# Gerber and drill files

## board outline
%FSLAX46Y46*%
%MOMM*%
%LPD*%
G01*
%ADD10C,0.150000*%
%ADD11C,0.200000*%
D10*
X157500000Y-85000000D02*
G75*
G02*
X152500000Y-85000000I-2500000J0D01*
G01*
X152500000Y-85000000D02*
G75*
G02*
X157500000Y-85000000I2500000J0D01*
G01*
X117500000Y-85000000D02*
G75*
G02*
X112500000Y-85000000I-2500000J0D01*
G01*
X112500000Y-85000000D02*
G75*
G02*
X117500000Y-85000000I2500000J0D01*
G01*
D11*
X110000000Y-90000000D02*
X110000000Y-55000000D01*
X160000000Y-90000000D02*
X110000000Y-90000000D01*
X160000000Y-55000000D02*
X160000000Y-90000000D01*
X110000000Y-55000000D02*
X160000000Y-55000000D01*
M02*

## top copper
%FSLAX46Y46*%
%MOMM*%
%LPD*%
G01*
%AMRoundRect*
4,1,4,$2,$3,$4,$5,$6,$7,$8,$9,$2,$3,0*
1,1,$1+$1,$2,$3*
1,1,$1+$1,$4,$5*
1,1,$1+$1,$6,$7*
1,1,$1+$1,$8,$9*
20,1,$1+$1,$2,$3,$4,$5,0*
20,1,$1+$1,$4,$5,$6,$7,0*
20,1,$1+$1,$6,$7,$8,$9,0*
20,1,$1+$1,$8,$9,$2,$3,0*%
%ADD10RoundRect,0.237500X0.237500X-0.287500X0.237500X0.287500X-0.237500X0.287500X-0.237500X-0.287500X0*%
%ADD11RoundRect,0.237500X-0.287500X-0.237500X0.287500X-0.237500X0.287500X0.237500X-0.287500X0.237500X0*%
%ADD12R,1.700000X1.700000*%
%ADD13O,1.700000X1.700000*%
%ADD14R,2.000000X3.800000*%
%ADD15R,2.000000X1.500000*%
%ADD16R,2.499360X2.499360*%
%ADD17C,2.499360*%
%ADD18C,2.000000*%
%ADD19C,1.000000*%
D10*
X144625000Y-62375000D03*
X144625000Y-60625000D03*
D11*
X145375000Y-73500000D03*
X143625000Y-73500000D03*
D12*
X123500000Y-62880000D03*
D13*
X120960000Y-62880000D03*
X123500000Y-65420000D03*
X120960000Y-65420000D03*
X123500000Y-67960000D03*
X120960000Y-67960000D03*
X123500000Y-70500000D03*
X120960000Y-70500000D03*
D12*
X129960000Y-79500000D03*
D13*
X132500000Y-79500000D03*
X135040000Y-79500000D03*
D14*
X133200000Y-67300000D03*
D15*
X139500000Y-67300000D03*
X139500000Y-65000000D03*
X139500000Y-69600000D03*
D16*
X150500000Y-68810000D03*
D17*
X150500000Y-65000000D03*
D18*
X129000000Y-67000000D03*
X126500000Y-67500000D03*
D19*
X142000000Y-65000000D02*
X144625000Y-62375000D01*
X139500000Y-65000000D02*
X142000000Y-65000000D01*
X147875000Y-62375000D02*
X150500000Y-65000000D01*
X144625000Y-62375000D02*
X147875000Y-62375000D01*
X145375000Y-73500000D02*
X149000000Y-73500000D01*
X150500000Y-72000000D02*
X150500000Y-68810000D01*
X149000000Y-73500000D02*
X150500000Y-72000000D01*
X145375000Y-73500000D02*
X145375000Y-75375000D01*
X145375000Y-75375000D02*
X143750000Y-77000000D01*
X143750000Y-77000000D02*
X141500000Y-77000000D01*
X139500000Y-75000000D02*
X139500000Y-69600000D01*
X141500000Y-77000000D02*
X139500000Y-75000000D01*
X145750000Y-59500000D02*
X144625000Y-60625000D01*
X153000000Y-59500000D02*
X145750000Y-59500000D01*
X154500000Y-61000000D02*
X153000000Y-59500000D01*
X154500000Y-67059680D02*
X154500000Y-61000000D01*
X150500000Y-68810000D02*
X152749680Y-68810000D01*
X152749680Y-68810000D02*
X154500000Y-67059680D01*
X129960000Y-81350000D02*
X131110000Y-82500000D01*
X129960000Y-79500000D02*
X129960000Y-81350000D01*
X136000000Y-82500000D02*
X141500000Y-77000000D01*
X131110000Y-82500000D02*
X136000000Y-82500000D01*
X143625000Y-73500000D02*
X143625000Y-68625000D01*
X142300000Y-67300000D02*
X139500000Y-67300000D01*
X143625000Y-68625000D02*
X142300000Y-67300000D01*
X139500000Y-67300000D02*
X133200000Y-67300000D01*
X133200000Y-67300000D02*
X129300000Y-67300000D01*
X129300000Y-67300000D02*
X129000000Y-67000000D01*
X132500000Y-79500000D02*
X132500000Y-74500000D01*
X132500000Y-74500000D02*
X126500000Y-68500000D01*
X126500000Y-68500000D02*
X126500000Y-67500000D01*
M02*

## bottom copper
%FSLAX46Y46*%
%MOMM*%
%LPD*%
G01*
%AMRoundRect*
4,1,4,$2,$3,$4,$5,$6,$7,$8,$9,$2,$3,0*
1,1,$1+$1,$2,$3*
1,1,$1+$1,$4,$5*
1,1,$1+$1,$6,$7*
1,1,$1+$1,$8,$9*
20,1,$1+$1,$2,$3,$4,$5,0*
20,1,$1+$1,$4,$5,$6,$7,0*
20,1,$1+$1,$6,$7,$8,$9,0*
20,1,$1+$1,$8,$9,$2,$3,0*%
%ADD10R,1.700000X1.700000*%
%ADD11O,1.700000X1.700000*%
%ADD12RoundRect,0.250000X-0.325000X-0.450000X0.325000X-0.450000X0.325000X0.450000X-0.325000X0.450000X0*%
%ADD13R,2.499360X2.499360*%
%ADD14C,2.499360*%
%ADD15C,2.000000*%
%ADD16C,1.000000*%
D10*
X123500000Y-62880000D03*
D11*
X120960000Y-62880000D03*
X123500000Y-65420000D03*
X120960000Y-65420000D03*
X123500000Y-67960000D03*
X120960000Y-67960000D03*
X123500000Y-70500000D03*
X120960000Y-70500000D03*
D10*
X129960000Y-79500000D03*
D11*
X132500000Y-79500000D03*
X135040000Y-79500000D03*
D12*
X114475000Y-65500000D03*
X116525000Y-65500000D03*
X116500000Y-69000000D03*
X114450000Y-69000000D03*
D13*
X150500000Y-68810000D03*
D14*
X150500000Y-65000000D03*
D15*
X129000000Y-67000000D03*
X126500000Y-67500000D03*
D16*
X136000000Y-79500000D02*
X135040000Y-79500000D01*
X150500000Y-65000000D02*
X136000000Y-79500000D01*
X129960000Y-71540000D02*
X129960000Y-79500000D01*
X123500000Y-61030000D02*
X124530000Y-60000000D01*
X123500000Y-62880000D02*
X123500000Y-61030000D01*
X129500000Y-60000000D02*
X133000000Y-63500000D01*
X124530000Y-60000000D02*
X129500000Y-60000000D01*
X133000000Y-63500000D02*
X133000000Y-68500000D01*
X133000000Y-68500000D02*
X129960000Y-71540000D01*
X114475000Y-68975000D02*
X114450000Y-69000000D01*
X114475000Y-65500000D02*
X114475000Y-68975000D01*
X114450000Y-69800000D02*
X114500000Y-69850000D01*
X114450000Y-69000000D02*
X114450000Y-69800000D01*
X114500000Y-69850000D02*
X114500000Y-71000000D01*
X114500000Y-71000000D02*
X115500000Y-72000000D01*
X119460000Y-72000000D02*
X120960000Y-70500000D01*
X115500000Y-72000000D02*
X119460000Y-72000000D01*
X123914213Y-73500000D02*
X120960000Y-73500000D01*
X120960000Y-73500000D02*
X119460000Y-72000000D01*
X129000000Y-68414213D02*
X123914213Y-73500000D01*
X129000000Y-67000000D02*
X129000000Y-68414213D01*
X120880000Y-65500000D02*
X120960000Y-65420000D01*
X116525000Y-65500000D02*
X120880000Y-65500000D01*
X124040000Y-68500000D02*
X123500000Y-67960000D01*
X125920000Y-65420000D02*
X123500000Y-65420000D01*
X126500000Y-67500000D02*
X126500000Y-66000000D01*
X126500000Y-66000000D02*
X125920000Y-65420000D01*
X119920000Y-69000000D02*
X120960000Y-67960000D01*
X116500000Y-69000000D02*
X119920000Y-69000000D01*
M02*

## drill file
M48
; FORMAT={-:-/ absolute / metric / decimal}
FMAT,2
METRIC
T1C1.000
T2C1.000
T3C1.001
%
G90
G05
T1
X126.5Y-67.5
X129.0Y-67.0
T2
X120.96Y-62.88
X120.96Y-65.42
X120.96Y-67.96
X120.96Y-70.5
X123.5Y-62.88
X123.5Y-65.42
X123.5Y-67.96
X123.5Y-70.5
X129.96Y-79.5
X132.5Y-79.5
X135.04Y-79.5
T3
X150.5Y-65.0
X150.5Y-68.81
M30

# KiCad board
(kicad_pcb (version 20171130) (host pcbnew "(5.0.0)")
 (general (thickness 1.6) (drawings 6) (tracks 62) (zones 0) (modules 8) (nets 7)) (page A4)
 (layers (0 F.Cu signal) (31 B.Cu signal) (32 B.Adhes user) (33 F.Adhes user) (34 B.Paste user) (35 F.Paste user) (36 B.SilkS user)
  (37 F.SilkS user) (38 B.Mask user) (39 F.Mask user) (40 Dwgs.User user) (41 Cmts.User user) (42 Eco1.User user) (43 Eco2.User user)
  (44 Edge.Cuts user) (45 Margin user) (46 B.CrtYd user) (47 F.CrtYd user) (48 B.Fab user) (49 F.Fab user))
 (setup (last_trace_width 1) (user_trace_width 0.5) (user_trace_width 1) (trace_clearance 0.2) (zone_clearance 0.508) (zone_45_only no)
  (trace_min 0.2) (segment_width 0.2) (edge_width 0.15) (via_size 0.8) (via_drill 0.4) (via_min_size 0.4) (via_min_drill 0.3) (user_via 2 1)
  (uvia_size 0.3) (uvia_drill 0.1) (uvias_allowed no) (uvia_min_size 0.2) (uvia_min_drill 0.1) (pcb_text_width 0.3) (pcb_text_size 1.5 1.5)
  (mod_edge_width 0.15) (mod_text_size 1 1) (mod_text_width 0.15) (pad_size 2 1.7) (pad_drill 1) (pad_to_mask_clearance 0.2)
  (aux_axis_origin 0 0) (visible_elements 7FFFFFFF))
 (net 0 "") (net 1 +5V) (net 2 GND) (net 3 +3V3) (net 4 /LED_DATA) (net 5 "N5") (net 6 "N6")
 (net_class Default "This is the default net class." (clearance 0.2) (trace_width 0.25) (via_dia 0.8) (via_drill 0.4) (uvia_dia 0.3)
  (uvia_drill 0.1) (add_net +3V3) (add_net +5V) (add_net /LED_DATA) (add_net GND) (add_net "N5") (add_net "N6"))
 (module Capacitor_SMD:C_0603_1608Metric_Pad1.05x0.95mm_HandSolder (layer F.Cu) (at 144.625 61.5 90)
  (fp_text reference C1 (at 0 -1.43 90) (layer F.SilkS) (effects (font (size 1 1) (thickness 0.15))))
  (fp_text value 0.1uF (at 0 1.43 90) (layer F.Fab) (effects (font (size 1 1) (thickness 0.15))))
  (pad 1 smd roundrect (at -0.875 0 90) (size 1.05 0.95) (layers F.Cu F.Paste F.Mask) (roundrect_rratio 0.25) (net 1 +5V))
  (pad 2 smd roundrect (at 0.875 0 90) (size 1.05 0.95) (layers F.Cu F.Paste F.Mask) (roundrect_rratio 0.25) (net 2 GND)))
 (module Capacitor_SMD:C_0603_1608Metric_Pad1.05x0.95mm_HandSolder (layer F.Cu) (at 144.5 73.5)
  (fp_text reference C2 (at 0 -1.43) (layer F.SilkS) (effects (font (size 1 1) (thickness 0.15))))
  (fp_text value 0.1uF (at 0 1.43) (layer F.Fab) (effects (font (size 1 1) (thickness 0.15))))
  (pad 2 smd roundrect (at 0.875 0) (size 1.05 0.95) (layers F.Cu F.Paste F.Mask) (roundrect_rratio 0.25) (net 2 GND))
  (pad 1 smd roundrect (at -0.875 0) (size 1.05 0.95) (layers F.Cu F.Paste F.Mask) (roundrect_rratio 0.25) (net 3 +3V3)))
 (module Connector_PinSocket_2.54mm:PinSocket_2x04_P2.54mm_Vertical (layer F.Cu) (at 123.5 62.88)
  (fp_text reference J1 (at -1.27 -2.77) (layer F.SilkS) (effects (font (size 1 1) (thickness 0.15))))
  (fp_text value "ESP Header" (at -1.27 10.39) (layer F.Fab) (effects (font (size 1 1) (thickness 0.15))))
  (pad 1 thru_hole rect (at 0 0) (size 1.7 1.7) (drill 1) (layers *.Cu *.Mask) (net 2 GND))
  (pad 2 thru_hole oval (at -2.54 0) (size 1.7 1.7) (drill 1) (layers *.Cu *.Mask))
  (pad 3 thru_hole oval (at 0 2.54) (size 1.7 1.7) (drill 1) (layers *.Cu *.Mask) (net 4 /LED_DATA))
  (pad 4 thru_hole oval (at -2.54 2.54) (size 1.7 1.7) (drill 1) (layers *.Cu *.Mask) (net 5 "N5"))
  (pad 5 thru_hole oval (at 0 5.08) (size 1.7 1.7) (drill 1) (layers *.Cu *.Mask))
  (pad 6 thru_hole oval (at -2.54 5.08) (size 1.7 1.7) (drill 1) (layers *.Cu *.Mask) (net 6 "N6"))
  (pad 7 thru_hole oval (at 0 7.62) (size 1.7 1.7) (drill 1) (layers *.Cu *.Mask))
  (pad 8 thru_hole oval (at -2.54 7.62) (size 1.7 1.7) (drill 1) (layers *.Cu *.Mask) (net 3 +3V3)))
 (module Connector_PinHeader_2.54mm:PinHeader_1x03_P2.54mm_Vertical (layer F.Cu) (at 129.96 79.5 90)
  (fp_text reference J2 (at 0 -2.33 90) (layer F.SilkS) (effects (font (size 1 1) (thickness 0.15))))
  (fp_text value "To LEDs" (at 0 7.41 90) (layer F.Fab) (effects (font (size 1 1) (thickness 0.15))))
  (pad 1 thru_hole rect (at 0 0 90) (size 1.7 1.7) (drill 1) (layers *.Cu *.Mask) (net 2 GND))
  (pad 2 thru_hole oval (at 0 2.54 90) (size 1.7 1.7) (drill 1) (layers *.Cu *.Mask) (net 4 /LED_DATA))
  (pad 3 thru_hole oval (at 0 5.08 90) (size 1.7 1.7) (drill 1) (layers *.Cu *.Mask) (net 1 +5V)))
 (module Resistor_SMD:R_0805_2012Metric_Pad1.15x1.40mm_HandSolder (layer B.Cu) (at 115.5 65.5)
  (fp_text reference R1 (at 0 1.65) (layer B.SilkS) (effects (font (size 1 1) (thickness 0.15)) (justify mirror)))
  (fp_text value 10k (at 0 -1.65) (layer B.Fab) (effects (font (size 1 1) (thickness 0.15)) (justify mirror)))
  (pad 1 smd roundrect (at -1.025 0) (size 1.15 1.4) (layers B.Cu B.Paste B.Mask) (roundrect_rratio 0.217391) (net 3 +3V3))
  (pad 2 smd roundrect (at 1.025 0) (size 1.15 1.4) (layers B.Cu B.Paste B.Mask) (roundrect_rratio 0.217391) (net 5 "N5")))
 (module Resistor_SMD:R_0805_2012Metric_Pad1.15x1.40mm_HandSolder (layer B.Cu) (at 115.475 69)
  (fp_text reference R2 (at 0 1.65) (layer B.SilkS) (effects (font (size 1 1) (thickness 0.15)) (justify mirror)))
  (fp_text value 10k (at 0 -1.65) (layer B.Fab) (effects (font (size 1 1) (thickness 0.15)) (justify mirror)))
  (pad 2 smd roundrect (at 1.025 0) (size 1.15 1.4) (layers B.Cu B.Paste B.Mask) (roundrect_rratio 0.217391) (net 6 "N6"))
  (pad 1 smd roundrect (at -1.025 0) (size 1.15 1.4) (layers B.Cu B.Paste B.Mask) (roundrect_rratio 0.217391) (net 3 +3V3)))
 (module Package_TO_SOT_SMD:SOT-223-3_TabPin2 (layer F.Cu) (at 136.35 67.3 180)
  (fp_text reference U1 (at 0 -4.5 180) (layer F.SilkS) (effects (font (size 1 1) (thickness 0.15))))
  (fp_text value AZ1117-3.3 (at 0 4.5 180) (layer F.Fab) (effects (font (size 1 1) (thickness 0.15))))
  (pad 2 smd rect (at 3.15 0 180) (size 2 3.8) (layers F.Cu F.Paste F.Mask) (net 3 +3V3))
  (pad 2 smd rect (at -3.15 0 180) (size 2 1.5) (layers F.Cu F.Paste F.Mask) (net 3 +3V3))
  (pad 3 smd rect (at -3.15 2.3 180) (size 2 1.5) (layers F.Cu F.Paste F.Mask) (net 1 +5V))
  (pad 1 smd rect (at -3.15 -2.3 180) (size 2 1.5) (layers F.Cu F.Paste F.Mask) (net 2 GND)))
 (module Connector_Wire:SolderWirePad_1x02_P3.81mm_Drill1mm (layer F.Cu) (at 150.5 68.81 90)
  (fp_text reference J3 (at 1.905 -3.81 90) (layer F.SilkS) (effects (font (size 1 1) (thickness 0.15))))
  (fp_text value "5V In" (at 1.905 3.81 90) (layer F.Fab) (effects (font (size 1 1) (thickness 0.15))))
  (pad 1 thru_hole rect (at 0 0 90) (size 2.49936 2.49936) (drill 1.00076) (layers *.Cu *.Mask) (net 2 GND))
  (pad 2 thru_hole circle (at 3.81 0 90) (size 2.49936 2.49936) (drill 1.00076) (layers *.Cu *.Mask) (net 1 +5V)))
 (gr_circle (center 155 85) (end 157.5 85) (layer Edge.Cuts) (width 0.15))
 (gr_circle (center 115 85) (end 117.5 85) (layer Edge.Cuts) (width 0.15))
 (gr_line (start 110 90) (end 110 55) (layer Edge.Cuts) (width 0.2))
 (gr_line (start 160 90) (end 110 90) (layer Edge.Cuts) (width 0.2))
 (gr_line (start 160 55) (end 160 90) (layer Edge.Cuts) (width 0.2))
 (gr_line (start 110 55) (end 160 55) (layer Edge.Cuts) (width 0.2))
 (segment (start 142 65) (end 144.625 62.375) (width 1) (layer F.Cu) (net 1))
 (segment (start 139.5 65) (end 142 65) (width 1) (layer F.Cu) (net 1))
 (segment (start 147.875 62.375) (end 150.5 65) (width 1) (layer F.Cu) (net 1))
 (segment (start 144.625 62.375) (end 147.875 62.375) (width 1) (layer F.Cu) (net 1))
 (segment (start 136 79.5) (end 135.04 79.5) (width 1) (layer B.Cu) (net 1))
 (segment (start 150.5 65) (end 136 79.5) (width 1) (layer B.Cu) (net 1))
 (segment (start 145.375 73.5) (end 149 73.5) (width 1) (layer F.Cu) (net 2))
 (segment (start 150.5 72) (end 150.5 68.81) (width 1) (layer F.Cu) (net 2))
 (segment (start 149 73.5) (end 150.5 72) (width 1) (layer F.Cu) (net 2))
 (segment (start 145.375 73.5) (end 145.375 75.375) (width 1) (layer F.Cu) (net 2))
 (segment (start 145.375 75.375) (end 143.75 77) (width 1) (layer F.Cu) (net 2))
 (segment (start 143.75 77) (end 141.5 77) (width 1) (layer F.Cu) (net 2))
 (segment (start 139.5 75) (end 139.5 69.6) (width 1) (layer F.Cu) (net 2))
 (segment (start 141.5 77) (end 139.5 75) (width 1) (layer F.Cu) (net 2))
 (segment (start 145.75 59.5) (end 144.625 60.625) (width 1) (layer F.Cu) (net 2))
 (segment (start 153 59.5) (end 145.75 59.5) (width 1) (layer F.Cu) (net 2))
 (segment (start 154.5 61) (end 153 59.5) (width 1) (layer F.Cu) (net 2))
 (segment (start 154.5 67.05968) (end 154.5 61) (width 1) (layer F.Cu) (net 2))
 (segment (start 150.5 68.81) (end 152.74968 68.81) (width 1) (layer F.Cu) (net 2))
 (segment (start 152.74968 68.81) (end 154.5 67.05968) (width 1) (layer F.Cu) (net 2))
 (segment (start 129.96 81.35) (end 131.11 82.5) (width 1) (layer F.Cu) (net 2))
 (segment (start 129.96 79.5) (end 129.96 81.35) (width 1) (layer F.Cu) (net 2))
 (segment (start 136 82.5) (end 141.5 77) (width 1) (layer F.Cu) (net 2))
 (segment (start 131.11 82.5) (end 136 82.5) (width 1) (layer F.Cu) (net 2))
 (segment (start 129.96 71.54) (end 129.96 79.5) (width 1) (layer B.Cu) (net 2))
 (segment (start 123.5 61.03) (end 124.53 60) (width 1) (layer B.Cu) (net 2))
 (segment (start 123.5 62.88) (end 123.5 61.03) (width 1) (layer B.Cu) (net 2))
 (segment (start 129.5 60) (end 133 63.5) (width 1) (layer B.Cu) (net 2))
 (segment (start 124.53 60) (end 129.5 60) (width 1) (layer B.Cu) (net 2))
 (segment (start 133 63.5) (end 133 68.5) (width 1) (layer B.Cu) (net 2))
 (segment (start 133 68.5) (end 129.96 71.54) (width 1) (layer B.Cu) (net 2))
 (segment (start 114.475 68.975) (end 114.45 69) (width 1) (layer B.Cu) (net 3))
 (segment (start 114.475 65.5) (end 114.475 68.975) (width 1) (layer B.Cu) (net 3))
 (segment (start 114.45 69.8) (end 114.5 69.85) (width 1) (layer B.Cu) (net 3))
 (segment (start 114.45 69) (end 114.45 69.8) (width 1) (layer B.Cu) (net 3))
 (segment (start 114.5 69.85) (end 114.5 71) (width 1) (layer B.Cu) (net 3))
 (segment (start 114.5 71) (end 115.5 72) (width 1) (layer B.Cu) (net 3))
 (segment (start 119.46 72) (end 120.96 70.5) (width 1) (layer B.Cu) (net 3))
 (segment (start 115.5 72) (end 119.46 72) (width 1) (layer B.Cu) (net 3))
 (segment (start 143.625 73.5) (end 143.625 68.625) (width 1) (layer F.Cu) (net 3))
 (segment (start 142.3 67.3) (end 139.5 67.3) (width 1) (layer F.Cu) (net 3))
 (segment (start 143.625 68.625) (end 142.3 67.3) (width 1) (layer F.Cu) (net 3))
 (segment (start 139.5 67.3) (end 133.2 67.3) (width 1) (layer F.Cu) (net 3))
 (via (at 129 67) (size 2) (drill 1) (layers F.Cu B.Cu) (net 3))
 (segment (start 133.2 67.3) (end 129.3 67.3) (width 1) (layer F.Cu) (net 3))
 (segment (start 129.3 67.3) (end 129 67) (width 1) (layer F.Cu) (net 3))
 (segment (start 123.914213 73.5) (end 120.96 73.5) (width 1) (layer B.Cu) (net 3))
 (segment (start 120.96 73.5) (end 119.46 72) (width 1) (layer B.Cu) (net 3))
 (segment (start 129 68.414213) (end 123.914213 73.5) (width 1) (layer B.Cu) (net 3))
 (segment (start 129 67) (end 129 68.414213) (width 1) (layer B.Cu) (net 3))
 (segment (start 120.88 65.5) (end 120.96 65.42) (width 1) (layer B.Cu) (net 5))
 (segment (start 116.525 65.5) (end 120.88 65.5) (width 1) (layer B.Cu) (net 5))
 (segment (start 132.5 79.5) (end 132.5 74.5) (width 1) (layer F.Cu) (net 4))
 (segment (start 132.5 74.5) (end 126.5 68.5) (width 1) (layer F.Cu) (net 4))
 (segment (start 124.04 68.5) (end 123.5 67.96) (width 1) (layer B.Cu) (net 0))
 (via (at 126.5 67.5) (size 2) (drill 1) (layers F.Cu B.Cu) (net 4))
 (segment (start 126.5 68.5) (end 126.5 67.5) (width 1) (layer F.Cu) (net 4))
 (segment (start 125.92 65.42) (end 123.5 65.42) (width 1) (layer B.Cu) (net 4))
 (segment (start 126.5 67.5) (end 126.5 66) (width 1) (layer B.Cu) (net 4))
 (segment (start 126.5 66) (end 125.92 65.42) (width 1) (layer B.Cu) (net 4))
 (segment (start 119.92 69) (end 120.96 67.96) (width 1) (layer B.Cu) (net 6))
 (segment (start 116.5 69) (end 119.92 69) (width 1) (layer B.Cu) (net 6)))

